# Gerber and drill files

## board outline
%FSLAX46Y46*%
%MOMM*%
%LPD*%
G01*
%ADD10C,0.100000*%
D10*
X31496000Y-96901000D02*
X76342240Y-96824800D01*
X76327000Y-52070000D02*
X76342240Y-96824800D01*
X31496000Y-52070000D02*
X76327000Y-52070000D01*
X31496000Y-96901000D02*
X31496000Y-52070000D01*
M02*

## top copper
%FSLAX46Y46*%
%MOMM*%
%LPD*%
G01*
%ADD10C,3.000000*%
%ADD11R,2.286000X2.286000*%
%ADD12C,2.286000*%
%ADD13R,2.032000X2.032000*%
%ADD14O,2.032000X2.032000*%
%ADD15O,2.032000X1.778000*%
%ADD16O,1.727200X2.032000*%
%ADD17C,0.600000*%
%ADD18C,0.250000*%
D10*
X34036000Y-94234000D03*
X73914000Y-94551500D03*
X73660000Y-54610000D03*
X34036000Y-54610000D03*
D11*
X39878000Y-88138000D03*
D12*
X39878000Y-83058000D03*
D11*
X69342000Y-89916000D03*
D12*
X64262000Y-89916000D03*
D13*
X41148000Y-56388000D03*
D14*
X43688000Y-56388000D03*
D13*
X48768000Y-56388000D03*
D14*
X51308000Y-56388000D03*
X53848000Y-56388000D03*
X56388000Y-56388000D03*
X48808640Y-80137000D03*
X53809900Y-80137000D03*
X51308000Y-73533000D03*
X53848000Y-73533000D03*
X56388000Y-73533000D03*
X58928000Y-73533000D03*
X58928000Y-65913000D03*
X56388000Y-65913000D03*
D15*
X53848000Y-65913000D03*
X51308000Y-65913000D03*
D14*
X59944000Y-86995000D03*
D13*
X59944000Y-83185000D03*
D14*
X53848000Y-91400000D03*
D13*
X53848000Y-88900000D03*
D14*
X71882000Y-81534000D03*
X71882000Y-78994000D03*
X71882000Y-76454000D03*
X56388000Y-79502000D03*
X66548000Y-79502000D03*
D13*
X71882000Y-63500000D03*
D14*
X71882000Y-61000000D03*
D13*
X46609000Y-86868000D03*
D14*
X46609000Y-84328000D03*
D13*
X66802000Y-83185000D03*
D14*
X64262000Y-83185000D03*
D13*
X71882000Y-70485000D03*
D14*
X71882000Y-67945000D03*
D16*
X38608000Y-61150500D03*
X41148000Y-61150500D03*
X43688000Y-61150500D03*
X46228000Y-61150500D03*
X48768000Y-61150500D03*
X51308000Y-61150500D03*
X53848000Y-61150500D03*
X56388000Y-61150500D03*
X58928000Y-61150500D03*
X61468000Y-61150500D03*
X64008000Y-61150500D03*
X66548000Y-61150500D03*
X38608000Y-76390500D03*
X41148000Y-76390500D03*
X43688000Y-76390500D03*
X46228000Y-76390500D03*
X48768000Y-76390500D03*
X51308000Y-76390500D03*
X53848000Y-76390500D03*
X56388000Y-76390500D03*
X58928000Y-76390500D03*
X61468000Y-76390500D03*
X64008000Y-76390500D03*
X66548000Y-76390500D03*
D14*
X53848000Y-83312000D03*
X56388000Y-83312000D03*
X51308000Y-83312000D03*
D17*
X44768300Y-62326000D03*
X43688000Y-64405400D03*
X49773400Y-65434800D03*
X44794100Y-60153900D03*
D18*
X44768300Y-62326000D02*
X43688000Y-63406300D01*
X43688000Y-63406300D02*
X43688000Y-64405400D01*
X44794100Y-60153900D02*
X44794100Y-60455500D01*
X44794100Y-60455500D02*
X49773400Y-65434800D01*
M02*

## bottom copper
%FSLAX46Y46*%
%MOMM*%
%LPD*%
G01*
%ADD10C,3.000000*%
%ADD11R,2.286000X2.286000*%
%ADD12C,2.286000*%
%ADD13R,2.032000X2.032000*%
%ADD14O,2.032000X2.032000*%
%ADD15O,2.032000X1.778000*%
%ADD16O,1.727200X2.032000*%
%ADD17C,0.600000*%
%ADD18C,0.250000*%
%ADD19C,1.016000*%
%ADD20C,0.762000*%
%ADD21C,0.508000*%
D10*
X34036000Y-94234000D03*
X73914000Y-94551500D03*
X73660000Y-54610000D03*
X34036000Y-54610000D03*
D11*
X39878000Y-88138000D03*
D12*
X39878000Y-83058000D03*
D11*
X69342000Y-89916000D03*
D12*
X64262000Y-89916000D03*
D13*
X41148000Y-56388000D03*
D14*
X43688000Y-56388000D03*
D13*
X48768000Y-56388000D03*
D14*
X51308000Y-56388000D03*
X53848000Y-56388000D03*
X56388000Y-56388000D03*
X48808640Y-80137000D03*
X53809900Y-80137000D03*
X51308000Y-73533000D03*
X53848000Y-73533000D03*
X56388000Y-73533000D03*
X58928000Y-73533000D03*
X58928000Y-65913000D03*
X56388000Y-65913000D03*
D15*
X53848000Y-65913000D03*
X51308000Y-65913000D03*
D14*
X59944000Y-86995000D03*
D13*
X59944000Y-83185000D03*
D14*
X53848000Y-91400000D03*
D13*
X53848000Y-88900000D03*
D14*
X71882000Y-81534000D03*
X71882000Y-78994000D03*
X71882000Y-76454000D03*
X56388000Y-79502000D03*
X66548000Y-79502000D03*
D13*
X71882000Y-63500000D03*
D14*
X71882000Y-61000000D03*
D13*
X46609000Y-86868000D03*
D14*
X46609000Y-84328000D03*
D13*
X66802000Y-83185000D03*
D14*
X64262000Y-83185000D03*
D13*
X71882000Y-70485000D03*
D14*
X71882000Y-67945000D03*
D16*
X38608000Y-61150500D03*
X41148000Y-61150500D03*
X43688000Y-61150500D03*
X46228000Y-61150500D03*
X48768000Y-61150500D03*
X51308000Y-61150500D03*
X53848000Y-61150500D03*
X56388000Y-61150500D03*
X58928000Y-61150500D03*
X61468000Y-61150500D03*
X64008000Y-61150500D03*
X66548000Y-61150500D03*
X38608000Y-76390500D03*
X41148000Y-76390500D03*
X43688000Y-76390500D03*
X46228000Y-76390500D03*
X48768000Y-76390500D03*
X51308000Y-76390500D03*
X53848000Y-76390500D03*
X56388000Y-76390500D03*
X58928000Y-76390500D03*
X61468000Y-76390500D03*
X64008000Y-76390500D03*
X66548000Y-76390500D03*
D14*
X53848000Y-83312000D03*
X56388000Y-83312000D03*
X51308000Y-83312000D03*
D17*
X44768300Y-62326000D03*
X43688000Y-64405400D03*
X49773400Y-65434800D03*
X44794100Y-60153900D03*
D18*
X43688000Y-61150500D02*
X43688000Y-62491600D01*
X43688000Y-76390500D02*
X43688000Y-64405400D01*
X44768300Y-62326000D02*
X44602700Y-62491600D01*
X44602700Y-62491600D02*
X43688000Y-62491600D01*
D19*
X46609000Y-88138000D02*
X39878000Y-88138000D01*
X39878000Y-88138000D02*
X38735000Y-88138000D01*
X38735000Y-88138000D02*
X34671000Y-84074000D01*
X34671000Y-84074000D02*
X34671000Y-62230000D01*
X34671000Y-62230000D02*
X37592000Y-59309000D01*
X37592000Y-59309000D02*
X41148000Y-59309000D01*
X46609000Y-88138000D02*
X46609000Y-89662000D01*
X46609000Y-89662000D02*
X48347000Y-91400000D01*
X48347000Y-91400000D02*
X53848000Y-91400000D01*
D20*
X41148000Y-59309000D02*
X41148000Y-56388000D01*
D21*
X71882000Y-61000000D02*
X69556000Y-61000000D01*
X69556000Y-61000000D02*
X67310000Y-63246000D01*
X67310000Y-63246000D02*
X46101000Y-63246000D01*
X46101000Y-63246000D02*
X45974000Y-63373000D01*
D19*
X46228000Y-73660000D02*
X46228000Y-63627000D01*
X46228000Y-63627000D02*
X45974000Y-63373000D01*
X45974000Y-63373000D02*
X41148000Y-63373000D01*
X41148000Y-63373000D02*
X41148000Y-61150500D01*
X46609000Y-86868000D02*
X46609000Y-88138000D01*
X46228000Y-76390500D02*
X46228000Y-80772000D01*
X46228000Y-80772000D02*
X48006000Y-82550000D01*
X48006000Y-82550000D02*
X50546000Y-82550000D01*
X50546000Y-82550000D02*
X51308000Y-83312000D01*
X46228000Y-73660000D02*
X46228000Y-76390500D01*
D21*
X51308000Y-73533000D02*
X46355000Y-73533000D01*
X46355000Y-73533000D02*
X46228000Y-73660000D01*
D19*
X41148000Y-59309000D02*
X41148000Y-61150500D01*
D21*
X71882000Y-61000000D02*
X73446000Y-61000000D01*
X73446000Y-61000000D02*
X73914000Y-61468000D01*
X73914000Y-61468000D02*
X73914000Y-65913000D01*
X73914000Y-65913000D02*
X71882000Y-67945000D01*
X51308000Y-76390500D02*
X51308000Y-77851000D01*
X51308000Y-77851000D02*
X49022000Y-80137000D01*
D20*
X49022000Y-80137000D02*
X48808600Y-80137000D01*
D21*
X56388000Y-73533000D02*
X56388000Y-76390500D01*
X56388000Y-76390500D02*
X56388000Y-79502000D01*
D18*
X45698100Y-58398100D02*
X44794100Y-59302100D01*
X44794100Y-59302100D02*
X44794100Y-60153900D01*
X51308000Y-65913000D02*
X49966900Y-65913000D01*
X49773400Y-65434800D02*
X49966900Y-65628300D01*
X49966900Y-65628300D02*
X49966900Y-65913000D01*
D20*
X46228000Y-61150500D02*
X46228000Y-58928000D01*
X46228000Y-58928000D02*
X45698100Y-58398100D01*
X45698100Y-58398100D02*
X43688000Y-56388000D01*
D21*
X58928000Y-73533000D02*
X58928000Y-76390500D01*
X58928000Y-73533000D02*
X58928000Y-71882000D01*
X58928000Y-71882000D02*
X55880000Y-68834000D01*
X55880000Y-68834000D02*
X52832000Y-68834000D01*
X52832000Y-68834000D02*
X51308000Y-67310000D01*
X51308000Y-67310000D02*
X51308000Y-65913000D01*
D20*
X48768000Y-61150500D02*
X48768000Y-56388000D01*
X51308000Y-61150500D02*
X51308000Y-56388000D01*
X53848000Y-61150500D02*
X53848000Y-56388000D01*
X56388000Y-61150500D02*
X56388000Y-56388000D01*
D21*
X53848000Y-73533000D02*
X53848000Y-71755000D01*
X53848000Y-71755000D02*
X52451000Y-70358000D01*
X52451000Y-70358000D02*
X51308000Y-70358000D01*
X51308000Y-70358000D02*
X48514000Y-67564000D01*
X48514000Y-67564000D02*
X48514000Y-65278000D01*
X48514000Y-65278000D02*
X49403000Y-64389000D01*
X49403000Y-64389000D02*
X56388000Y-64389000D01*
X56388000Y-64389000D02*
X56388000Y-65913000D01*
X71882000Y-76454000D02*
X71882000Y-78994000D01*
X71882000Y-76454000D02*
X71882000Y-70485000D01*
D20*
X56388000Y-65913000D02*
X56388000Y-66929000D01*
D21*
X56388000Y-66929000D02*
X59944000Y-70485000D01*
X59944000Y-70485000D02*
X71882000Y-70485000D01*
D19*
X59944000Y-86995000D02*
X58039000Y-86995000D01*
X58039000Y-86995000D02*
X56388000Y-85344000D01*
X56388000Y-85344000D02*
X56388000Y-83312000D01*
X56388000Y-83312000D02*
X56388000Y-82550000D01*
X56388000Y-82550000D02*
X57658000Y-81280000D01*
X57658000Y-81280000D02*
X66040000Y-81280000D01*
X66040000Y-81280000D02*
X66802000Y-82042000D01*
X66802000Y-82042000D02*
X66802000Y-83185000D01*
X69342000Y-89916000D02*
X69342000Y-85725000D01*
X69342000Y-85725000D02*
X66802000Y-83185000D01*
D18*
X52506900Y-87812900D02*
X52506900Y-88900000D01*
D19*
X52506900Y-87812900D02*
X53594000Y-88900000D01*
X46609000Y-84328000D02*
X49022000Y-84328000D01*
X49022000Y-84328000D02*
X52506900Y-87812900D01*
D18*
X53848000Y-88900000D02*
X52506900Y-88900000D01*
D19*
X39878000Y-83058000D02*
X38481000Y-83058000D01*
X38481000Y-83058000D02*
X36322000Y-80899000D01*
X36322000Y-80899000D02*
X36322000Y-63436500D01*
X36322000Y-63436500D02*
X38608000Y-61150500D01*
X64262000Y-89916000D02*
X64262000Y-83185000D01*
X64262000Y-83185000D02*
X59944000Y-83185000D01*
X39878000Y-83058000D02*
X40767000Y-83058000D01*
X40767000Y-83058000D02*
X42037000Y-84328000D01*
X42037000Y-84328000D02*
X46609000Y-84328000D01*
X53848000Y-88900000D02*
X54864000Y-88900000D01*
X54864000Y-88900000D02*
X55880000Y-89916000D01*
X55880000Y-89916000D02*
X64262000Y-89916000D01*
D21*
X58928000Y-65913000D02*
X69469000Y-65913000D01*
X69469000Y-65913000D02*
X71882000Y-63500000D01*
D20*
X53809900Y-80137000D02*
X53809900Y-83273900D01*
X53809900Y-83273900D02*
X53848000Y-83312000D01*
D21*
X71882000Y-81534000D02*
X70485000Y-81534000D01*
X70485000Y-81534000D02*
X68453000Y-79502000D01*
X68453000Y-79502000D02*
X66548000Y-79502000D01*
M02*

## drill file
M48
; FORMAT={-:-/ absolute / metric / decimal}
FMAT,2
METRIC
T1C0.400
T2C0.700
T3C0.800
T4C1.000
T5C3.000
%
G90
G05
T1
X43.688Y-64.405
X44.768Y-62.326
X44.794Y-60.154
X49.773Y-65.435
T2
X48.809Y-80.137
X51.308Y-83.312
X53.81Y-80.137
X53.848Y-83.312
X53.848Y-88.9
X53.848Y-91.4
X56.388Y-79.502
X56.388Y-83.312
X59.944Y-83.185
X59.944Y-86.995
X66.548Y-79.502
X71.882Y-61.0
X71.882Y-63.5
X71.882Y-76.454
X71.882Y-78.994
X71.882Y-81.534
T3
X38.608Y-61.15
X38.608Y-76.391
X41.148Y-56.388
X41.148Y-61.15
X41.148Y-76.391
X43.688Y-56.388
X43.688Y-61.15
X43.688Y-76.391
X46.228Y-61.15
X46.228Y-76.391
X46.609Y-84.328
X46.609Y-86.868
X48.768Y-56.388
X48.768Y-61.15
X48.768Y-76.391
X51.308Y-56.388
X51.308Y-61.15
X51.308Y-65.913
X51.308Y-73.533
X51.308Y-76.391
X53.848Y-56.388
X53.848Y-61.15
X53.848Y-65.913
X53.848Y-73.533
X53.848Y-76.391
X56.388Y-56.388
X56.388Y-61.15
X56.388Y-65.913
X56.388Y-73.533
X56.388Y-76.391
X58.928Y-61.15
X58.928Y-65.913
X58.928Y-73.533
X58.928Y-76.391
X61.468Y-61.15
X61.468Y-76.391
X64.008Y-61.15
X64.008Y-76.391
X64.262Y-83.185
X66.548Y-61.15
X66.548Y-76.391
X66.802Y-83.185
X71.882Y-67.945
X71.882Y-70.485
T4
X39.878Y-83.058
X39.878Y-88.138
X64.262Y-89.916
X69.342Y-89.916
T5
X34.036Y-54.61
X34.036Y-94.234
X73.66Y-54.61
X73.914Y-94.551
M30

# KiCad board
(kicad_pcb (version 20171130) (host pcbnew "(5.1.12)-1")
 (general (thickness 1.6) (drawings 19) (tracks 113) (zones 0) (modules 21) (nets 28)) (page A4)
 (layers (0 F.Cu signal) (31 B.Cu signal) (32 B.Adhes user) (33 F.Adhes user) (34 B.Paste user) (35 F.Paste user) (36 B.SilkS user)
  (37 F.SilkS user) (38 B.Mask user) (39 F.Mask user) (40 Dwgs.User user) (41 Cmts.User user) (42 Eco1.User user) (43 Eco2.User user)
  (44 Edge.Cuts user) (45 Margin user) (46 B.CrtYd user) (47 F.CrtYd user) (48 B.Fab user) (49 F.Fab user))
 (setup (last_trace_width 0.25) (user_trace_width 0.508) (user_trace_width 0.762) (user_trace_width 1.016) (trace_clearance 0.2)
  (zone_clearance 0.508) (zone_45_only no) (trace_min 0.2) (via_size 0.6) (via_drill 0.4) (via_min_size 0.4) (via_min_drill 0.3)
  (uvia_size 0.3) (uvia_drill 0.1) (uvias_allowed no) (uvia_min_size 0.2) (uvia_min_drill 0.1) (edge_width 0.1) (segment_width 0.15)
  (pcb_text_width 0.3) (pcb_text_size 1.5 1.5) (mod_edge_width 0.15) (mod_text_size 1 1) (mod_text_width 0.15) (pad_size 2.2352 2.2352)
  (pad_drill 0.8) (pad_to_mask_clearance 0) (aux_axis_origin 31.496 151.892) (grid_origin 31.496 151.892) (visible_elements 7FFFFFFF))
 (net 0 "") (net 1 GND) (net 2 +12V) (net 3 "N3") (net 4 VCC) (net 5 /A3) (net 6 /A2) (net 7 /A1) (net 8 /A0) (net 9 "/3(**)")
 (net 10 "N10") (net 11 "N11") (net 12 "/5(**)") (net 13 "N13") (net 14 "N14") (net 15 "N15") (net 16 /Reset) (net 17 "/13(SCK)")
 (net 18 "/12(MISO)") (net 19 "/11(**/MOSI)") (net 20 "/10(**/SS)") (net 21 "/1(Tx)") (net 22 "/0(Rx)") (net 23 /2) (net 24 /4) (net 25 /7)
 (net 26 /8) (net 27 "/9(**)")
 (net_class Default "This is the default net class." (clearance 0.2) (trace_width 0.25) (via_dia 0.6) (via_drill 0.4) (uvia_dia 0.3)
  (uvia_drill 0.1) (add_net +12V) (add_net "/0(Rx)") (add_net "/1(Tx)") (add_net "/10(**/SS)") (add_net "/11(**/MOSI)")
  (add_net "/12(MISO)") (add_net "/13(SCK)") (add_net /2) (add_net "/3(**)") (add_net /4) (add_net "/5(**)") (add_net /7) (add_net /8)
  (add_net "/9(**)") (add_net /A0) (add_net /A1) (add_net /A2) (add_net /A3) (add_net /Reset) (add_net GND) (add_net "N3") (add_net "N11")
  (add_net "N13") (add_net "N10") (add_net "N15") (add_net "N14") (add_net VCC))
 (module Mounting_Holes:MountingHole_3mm (layer F.Cu) (at 34.036 94.234)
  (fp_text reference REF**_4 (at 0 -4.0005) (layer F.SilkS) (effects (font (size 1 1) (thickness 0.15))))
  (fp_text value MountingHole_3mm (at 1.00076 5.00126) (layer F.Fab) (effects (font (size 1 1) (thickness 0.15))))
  (pad 1 thru_hole circle (at 0 0) (size 3 3) (drill 3) (layers *.Cu *.Mask)))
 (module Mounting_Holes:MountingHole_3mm (layer F.Cu) (at 73.914 94.5515)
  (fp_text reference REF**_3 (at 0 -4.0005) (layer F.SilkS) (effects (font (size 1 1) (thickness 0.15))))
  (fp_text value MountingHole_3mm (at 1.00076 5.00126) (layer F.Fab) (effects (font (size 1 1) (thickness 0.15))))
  (pad 1 thru_hole circle (at 0 0) (size 3 3) (drill 3) (layers *.Cu *.Mask)))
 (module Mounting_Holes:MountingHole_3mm (layer F.Cu) (at 73.66 54.61)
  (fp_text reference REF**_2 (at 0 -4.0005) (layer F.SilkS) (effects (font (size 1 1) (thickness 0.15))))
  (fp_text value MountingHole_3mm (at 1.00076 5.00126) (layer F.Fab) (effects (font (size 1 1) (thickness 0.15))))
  (pad 1 thru_hole circle (at 0 0) (size 3 3) (drill 3) (layers *.Cu *.Mask)))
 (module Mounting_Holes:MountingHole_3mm (layer F.Cu) (at 34.036 54.61)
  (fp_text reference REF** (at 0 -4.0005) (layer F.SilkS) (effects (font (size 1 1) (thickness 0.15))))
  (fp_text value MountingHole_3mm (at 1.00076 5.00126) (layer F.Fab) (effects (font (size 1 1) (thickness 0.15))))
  (pad 1 thru_hole circle (at 0 0) (size 3 3) (drill 3) (layers *.Cu *.Mask)))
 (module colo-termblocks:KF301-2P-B (layer F.Cu) (at 39.878 85.598 90)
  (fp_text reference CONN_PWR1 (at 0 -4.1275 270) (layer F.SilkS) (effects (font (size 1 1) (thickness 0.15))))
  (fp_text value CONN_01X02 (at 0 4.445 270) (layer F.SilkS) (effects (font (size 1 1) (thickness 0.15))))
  (pad 1 thru_hole rect (at -2.54 0 90) (size 2.286 2.286) (drill 1) (layers B.Cu B.Mask) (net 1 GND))
  (pad 2 thru_hole circle (at 2.54 0 90) (size 2.286 2.286) (drill 1) (layers B.Cu B.Mask) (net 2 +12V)))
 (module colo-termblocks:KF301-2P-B (layer F.Cu) (at 66.802 89.916 180)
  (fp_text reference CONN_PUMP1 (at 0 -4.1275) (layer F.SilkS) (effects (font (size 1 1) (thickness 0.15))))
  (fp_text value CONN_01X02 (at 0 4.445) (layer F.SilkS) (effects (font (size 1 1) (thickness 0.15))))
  (pad 1 thru_hole rect (at -2.54 0 180) (size 2.286 2.286) (drill 1) (layers B.Cu B.Mask) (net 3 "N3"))
  (pad 2 thru_hole circle (at 2.54 0 180) (size 2.286 2.286) (drill 1) (layers B.Cu B.Mask) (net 2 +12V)))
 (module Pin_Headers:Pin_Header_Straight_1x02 (layer F.Cu) (at 41.148 56.388 90)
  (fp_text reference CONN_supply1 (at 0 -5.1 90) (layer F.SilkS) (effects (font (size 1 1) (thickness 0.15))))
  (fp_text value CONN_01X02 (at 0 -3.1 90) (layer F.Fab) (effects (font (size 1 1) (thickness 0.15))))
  (pad 1 thru_hole rect (at 0 0 90) (size 2.032 2.032) (drill 0.8) (layers B.Cu B.Mask) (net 1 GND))
  (pad 2 thru_hole oval (at 0 2.54 90) (size 2.032 2.032) (drill 0.8) (layers B.Cu B.Mask) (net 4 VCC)))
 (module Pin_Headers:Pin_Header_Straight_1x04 (layer F.Cu) (at 48.768 56.388 90)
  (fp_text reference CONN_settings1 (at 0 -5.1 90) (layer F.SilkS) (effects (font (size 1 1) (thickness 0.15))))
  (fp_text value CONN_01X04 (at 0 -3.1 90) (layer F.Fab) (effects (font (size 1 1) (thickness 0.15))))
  (pad 1 thru_hole rect (at 0 0 90) (size 2.032 2.032) (drill 0.8) (layers B.Cu B.Mask) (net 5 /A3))
  (pad 2 thru_hole oval (at 0 2.54 90) (size 2.032 2.032) (drill 0.8) (layers B.Cu B.Mask) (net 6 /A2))
  (pad 3 thru_hole oval (at 0 5.08 90) (size 2.032 2.032) (drill 0.8) (layers B.Cu B.Mask) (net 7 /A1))
  (pad 4 thru_hole oval (at 0 7.62 90) (size 2.032 2.032) (drill 0.8) (layers B.Cu B.Mask) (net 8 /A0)))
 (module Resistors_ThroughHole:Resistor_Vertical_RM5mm (layer F.Cu) (at 51.308 80.137)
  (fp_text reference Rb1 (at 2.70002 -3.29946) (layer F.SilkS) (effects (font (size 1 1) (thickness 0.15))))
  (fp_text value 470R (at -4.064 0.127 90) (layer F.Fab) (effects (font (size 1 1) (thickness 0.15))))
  (pad 1 thru_hole oval (at -2.49936 0) (size 2.032 2.032) (drill 0.7) (layers B.Cu B.Mask) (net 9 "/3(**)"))
  (pad 2 thru_hole oval (at 2.5019 0) (size 2.032 2.032) (drill 0.7) (layers B.Cu B.Mask) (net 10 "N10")))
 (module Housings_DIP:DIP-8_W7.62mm (layer F.Cu) (at 51.308 73.533 90)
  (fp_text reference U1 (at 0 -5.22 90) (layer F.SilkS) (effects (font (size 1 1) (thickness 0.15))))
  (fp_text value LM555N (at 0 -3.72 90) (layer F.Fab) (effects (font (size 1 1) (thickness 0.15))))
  (pad 1 thru_hole oval (at 0 0 90) (size 2.032 2.032) (drill 0.8) (layers B.Cu B.Mask) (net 1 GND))
  (pad 2 thru_hole oval (at 0 2.54 90) (size 2.032 2.032) (drill 0.8) (layers B.Cu B.Mask) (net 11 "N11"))
  (pad 3 thru_hole oval (at 0 5.08 90) (size 2.032 2.032) (drill 0.8) (layers B.Cu B.Mask) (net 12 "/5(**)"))
  (pad 4 thru_hole oval (at 0 7.62 90) (size 2.032 2.032) (drill 0.8) (layers B.Cu B.Mask) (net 4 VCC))
  (pad 5 thru_hole oval (at 7.62 7.62 90) (size 2.032 2.032) (drill 0.8) (layers B.Cu B.Mask) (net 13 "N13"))
  (pad 6 thru_hole oval (at 7.62 5.08 90) (size 2.032 2.032) (drill 0.8) (layers B.Cu B.Mask) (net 11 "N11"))
  (pad 7 thru_hole oval (at 7.62 2.54 90) (size 1.778 2.032) (drill 0.8) (layers B.Cu B.Mask) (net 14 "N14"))
  (pad 8 thru_hole oval (at 7.62 0 90) (size 1.778 2.032) (drill 0.8) (layers B.Cu B.Mask) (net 4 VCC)))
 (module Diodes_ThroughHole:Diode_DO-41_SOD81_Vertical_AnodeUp (layer F.Cu) (at 59.944 83.185 270)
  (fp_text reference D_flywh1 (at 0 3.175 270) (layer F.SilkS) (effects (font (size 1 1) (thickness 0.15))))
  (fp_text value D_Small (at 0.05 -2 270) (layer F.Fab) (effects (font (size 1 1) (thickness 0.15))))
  (pad 2 thru_hole oval (at 3.81 0 270) (size 2.032 2.032) (drill 0.7) (layers B.Cu B.Mask) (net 3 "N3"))
  (pad 1 thru_hole rect (at 0 0 270) (size 2.032 2.032) (drill 0.7) (layers B.Cu B.Mask) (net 2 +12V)))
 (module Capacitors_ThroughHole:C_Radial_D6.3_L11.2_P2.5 (layer F.Cu) (at 53.848 88.9 270)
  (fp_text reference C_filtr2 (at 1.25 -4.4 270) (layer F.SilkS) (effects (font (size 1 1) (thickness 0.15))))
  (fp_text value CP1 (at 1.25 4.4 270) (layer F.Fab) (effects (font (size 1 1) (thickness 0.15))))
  (pad 2 thru_hole oval (at 2.5 0 270) (size 2.032 2.032) (drill 0.7) (layers B.Cu B.Mask) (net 1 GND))
  (pad 1 thru_hole rect (at 0 0 270) (size 2.032 2.032) (drill 0.7) (layers B.Cu B.Mask) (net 2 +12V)))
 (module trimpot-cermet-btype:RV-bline (layer F.Cu) (at 71.882 78.994 90)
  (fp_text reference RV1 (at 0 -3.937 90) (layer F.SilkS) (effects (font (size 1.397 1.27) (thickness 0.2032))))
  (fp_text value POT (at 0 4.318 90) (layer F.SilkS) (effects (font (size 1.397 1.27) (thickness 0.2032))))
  (pad 1 thru_hole oval (at -2.54 0 90) (size 2.032 2.032) (drill 0.7) (layers B.Cu B.Mask) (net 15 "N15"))
  (pad 2 thru_hole oval (at 0 0 90) (size 2.032 2.032) (drill 0.7) (layers B.Cu B.Mask) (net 11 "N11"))
  (pad 3 thru_hole oval (at 2.54 0 90) (size 2.032 2.032) (drill 0.7) (layers B.Cu B.Mask) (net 11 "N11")))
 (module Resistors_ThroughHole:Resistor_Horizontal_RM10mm (layer F.Cu) (at 61.468 79.502)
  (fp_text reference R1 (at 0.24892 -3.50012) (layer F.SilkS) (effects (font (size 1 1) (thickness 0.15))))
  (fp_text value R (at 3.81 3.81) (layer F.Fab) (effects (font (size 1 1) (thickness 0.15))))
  (pad 1 thru_hole oval (at -5.08 0) (size 2.032 2.032) (drill 0.7) (layers B.Cu B.Mask) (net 12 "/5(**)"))
  (pad 2 thru_hole oval (at 5.08 0) (size 2.032 2.032) (drill 0.7) (layers B.Cu B.Mask) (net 15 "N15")))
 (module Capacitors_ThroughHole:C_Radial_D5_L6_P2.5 (layer F.Cu) (at 71.882 63.5 90)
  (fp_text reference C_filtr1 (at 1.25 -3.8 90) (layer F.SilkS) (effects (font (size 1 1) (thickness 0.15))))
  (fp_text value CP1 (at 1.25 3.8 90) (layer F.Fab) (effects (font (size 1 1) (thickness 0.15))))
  (pad 1 thru_hole rect (at 0 0 90) (size 2.032 2.032) (drill 0.7) (layers B.Cu B.Mask) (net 13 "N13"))
  (pad 2 thru_hole oval (at 2.5 0 90) (size 2.032 2.032) (drill 0.7) (layers B.Cu B.Mask) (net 1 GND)))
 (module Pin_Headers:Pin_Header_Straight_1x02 (layer F.Cu) (at 46.609 86.868 180)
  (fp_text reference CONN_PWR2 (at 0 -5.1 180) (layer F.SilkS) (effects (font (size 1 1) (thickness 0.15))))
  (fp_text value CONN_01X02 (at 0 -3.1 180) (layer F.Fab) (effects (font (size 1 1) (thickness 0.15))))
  (pad 1 thru_hole rect (at 0 0 180) (size 2.032 2.032) (drill 0.8) (layers B.Cu B.Mask) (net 1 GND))
  (pad 2 thru_hole oval (at 0 2.54 180) (size 2.032 2.032) (drill 0.8) (layers B.Cu B.Mask) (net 2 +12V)))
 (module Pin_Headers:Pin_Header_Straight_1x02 (layer F.Cu) (at 66.802 83.185 270)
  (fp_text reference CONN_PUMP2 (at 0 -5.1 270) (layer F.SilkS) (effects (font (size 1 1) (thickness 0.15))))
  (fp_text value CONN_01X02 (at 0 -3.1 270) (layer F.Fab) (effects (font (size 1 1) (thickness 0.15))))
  (pad 1 thru_hole rect (at 0 0 270) (size 2.032 2.032) (drill 0.8) (layers B.Cu B.Mask) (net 3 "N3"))
  (pad 2 thru_hole oval (at 0 2.54 270) (size 2.032 2.032) (drill 0.8) (layers B.Cu B.Mask) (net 2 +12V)))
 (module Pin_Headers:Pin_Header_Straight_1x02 (layer F.Cu) (at 71.882 70.485 180)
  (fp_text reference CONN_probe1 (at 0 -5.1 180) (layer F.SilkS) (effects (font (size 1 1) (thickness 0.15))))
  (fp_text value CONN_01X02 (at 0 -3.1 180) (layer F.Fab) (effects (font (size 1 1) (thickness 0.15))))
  (pad 1 thru_hole rect (at 0 0 180) (size 2.032 2.032) (drill 0.8) (layers B.Cu B.Mask) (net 11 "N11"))
  (pad 2 thru_hole oval (at 0 2.54 180) (size 2.032 2.032) (drill 0.8) (layers B.Cu B.Mask) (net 1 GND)))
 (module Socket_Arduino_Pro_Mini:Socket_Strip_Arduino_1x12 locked (layer F.Cu) (at 38.608 61.1505)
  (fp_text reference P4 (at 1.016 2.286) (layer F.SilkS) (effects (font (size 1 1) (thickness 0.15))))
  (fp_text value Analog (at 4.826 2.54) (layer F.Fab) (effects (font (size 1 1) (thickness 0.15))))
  (pad 1 thru_hole oval (at 0 0) (size 1.7272 2.032) (drill 0.8) (layers B.Cu B.Mask) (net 2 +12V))
  (pad 2 thru_hole oval (at 2.54 0) (size 1.7272 2.032) (drill 0.8) (layers B.Cu B.Mask) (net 1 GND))
  (pad 3 thru_hole oval (at 5.08 0) (size 1.7272 2.032) (drill 0.8) (layers B.Cu B.Mask) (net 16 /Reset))
  (pad 4 thru_hole oval (at 7.62 0) (size 1.7272 2.032) (drill 0.8) (layers B.Cu B.Mask) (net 4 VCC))
  (pad 5 thru_hole oval (at 10.16 0) (size 1.7272 2.032) (drill 0.8) (layers B.Cu B.Mask) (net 5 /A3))
  (pad 6 thru_hole oval (at 12.7 0) (size 1.7272 2.032) (drill 0.8) (layers B.Cu B.Mask) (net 6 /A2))
  (pad 7 thru_hole oval (at 15.24 0) (size 1.7272 2.032) (drill 0.8) (layers B.Cu B.Mask) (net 7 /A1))
  (pad 8 thru_hole oval (at 17.78 0) (size 1.7272 2.032) (drill 0.8) (layers B.Cu B.Mask) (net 8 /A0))
  (pad 9 thru_hole oval (at 20.32 0) (size 1.7272 2.032) (drill 0.8) (layers B.Cu B.Mask) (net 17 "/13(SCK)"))
  (pad 10 thru_hole oval (at 22.86 0) (size 1.7272 2.032) (drill 0.8) (layers B.Cu B.Mask) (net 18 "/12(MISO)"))
  (pad 11 thru_hole oval (at 25.4 0) (size 1.7272 2.032) (drill 0.8) (layers B.Cu B.Mask) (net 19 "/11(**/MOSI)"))
  (pad 12 thru_hole oval (at 27.94 0) (size 1.7272 2.032) (drill 0.8) (layers B.Cu B.Mask) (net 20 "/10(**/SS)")))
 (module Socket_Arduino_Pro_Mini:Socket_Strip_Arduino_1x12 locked (layer F.Cu) (at 38.608 76.3905)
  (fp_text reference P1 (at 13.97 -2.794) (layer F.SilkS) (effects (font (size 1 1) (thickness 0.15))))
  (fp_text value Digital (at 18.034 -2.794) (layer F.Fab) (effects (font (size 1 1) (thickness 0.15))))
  (pad 1 thru_hole oval (at 0 0) (size 1.7272 2.032) (drill 0.8) (layers B.Cu B.Mask) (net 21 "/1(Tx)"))
  (pad 2 thru_hole oval (at 2.54 0) (size 1.7272 2.032) (drill 0.8) (layers B.Cu B.Mask) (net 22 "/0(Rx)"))
  (pad 3 thru_hole oval (at 5.08 0) (size 1.7272 2.032) (drill 0.8) (layers B.Cu B.Mask) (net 16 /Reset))
  (pad 4 thru_hole oval (at 7.62 0) (size 1.7272 2.032) (drill 0.8) (layers B.Cu B.Mask) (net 1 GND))
  (pad 5 thru_hole oval (at 10.16 0) (size 1.7272 2.032) (drill 0.8) (layers B.Cu B.Mask) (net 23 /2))
  (pad 6 thru_hole oval (at 12.7 0) (size 1.7272 2.032) (drill 0.8) (layers B.Cu B.Mask) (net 9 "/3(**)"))
  (pad 7 thru_hole oval (at 15.24 0) (size 1.7272 2.032) (drill 0.8) (layers B.Cu B.Mask) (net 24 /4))
  (pad 8 thru_hole oval (at 17.78 0) (size 1.7272 2.032) (drill 0.8) (layers B.Cu B.Mask) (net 12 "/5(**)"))
  (pad 9 thru_hole oval (at 20.32 0) (size 1.7272 2.032) (drill 0.8) (layers B.Cu B.Mask) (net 4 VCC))
  (pad 10 thru_hole oval (at 22.86 0) (size 1.7272 2.032) (drill 0.8) (layers B.Cu B.Mask) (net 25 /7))
  (pad 11 thru_hole oval (at 25.4 0) (size 1.7272 2.032) (drill 0.8) (layers B.Cu B.Mask) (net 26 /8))
  (pad 12 thru_hole oval (at 27.94 0) (size 1.7272 2.032) (drill 0.8) (layers B.Cu B.Mask) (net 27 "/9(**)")))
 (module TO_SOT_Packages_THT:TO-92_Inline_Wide (layer F.Cu) (at 51.308 83.312)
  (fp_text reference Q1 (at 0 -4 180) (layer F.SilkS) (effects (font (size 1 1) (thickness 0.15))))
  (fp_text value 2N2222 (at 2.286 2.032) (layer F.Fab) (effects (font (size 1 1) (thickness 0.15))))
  (pad 2 thru_hole oval (at 2.54 0) (size 2.032 2.032) (drill 0.7) (layers B.Cu B.Mask) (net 10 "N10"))
  (pad 3 thru_hole oval (at 5.08 0) (size 2.032 2.032) (drill 0.7) (layers B.Cu B.Mask) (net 3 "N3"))
  (pad 1 thru_hole oval (at 0 0) (size 2.032 2.032) (drill 0.7) (layers B.Cu B.Mask) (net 1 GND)))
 (gr_line (start 31.496 96.901) (end 76.34224 96.8248) (angle 90) (layer Edge.Cuts) (width 0.1))
 (gr_line (start 76.327 52.07) (end 76.34224 96.8248) (angle 90) (layer Edge.Cuts) (width 0.1))
 (gr_line (start 31.496 52.07) (end 76.327 52.07) (angle 90) (layer Edge.Cuts) (width 0.1))
 (gr_line (start 31.496 96.901) (end 31.496 52.07) (angle 90) (layer Edge.Cuts) (width 0.1))
 (segment (start 43.688 61.1505) (end 43.688 62.4916) (width 0.25) (layer B.Cu) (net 16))
 (segment (start 44.7683 62.326) (end 43.688 63.4063) (width 0.25) (layer F.Cu) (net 16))
 (segment (start 43.688 63.4063) (end 43.688 64.4054) (width 0.25) (layer F.Cu) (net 16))
 (segment (start 43.688 76.3905) (end 43.688 64.4054) (width 0.25) (layer B.Cu) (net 16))
 (segment (start 44.7683 62.326) (end 44.6027 62.4916) (width 0.25) (layer B.Cu) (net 16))
 (segment (start 44.6027 62.4916) (end 43.688 62.4916) (width 0.25) (layer B.Cu) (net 16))
 (via (at 44.7683 62.326) (size 0.6) (layers F.Cu B.Cu) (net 16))
 (via (at 43.688 64.4054) (size 0.6) (layers F.Cu B.Cu) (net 16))
 (segment (start 46.609 88.138) (end 39.878 88.138) (width 1.016) (layer B.Cu) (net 1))
 (segment (start 39.878 88.138) (end 38.735 88.138) (width 1.016) (layer B.Cu) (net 1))
 (segment (start 38.735 88.138) (end 34.671 84.074) (width 1.016) (layer B.Cu) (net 1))
 (segment (start 34.671 84.074) (end 34.671 62.23) (width 1.016) (layer B.Cu) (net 1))
 (segment (start 34.671 62.23) (end 37.592 59.309) (width 1.016) (layer B.Cu) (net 1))
 (segment (start 37.592 59.309) (end 41.148 59.309) (width 1.016) (layer B.Cu) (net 1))
 (segment (start 46.609 88.138) (end 46.609 89.662) (width 1.016) (layer B.Cu) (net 1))
 (segment (start 46.609 89.662) (end 48.347 91.4) (width 1.016) (layer B.Cu) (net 1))
 (segment (start 48.347 91.4) (end 53.848 91.4) (width 1.016) (layer B.Cu) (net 1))
 (segment (start 41.148 59.309) (end 41.148 56.388) (width 0.762) (layer B.Cu) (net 1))
 (segment (start 71.882 61) (end 69.556 61) (width 0.508) (layer B.Cu) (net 1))
 (segment (start 69.556 61) (end 67.31 63.246) (width 0.508) (layer B.Cu) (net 1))
 (segment (start 67.31 63.246) (end 46.101 63.246) (width 0.508) (layer B.Cu) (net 1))
 (segment (start 46.101 63.246) (end 45.974 63.373) (width 0.508) (layer B.Cu) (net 1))
 (segment (start 46.228 73.66) (end 46.228 63.627) (width 1.016) (layer B.Cu) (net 1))
 (segment (start 46.228 63.627) (end 45.974 63.373) (width 1.016) (layer B.Cu) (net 1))
 (segment (start 45.974 63.373) (end 41.148 63.373) (width 1.016) (layer B.Cu) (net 1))
 (segment (start 41.148 63.373) (end 41.148 61.1505) (width 1.016) (layer B.Cu) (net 1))
 (segment (start 46.609 86.868) (end 46.609 88.138) (width 1.016) (layer B.Cu) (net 1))
 (segment (start 46.228 76.3905) (end 46.228 80.772) (width 1.016) (layer B.Cu) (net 1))
 (segment (start 46.228 80.772) (end 48.006 82.55) (width 1.016) (layer B.Cu) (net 1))
 (segment (start 48.006 82.55) (end 50.546 82.55) (width 1.016) (layer B.Cu) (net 1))
 (segment (start 50.546 82.55) (end 51.308 83.312) (width 1.016) (layer B.Cu) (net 1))
 (segment (start 46.228 73.66) (end 46.228 76.3905) (width 1.016) (layer B.Cu) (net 1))
 (segment (start 51.308 73.533) (end 46.355 73.533) (width 0.508) (layer B.Cu) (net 1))
 (segment (start 46.355 73.533) (end 46.228 73.66) (width 0.508) (layer B.Cu) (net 1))
 (segment (start 41.148 59.309) (end 41.148 61.1505) (width 1.016) (layer B.Cu) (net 1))
 (segment (start 71.882 61) (end 73.446 61) (width 0.508) (layer B.Cu) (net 1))
 (segment (start 73.446 61) (end 73.914 61.468) (width 0.508) (layer B.Cu) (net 1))
 (segment (start 73.914 61.468) (end 73.914 65.913) (width 0.508) (layer B.Cu) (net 1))
 (segment (start 73.914 65.913) (end 71.882 67.945) (width 0.508) (layer B.Cu) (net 1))
 (segment (start 51.308 76.3905) (end 51.308 77.851) (width 0.508) (layer B.Cu) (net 9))
 (segment (start 51.308 77.851) (end 49.022 80.137) (width 0.508) (layer B.Cu) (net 9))
 (segment (start 49.022 80.137) (end 48.8086 80.137) (width 0.762) (layer B.Cu) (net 9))
 (segment (start 56.388 73.533) (end 56.388 76.3905) (width 0.508) (layer B.Cu) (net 12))
 (segment (start 56.388 76.3905) (end 56.388 79.502) (width 0.508) (layer B.Cu) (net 12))
 (segment (start 44.7941 60.1539) (end 44.7941 60.4555) (width 0.25) (layer F.Cu) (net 4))
 (segment (start 44.7941 60.4555) (end 49.7734 65.4348) (width 0.25) (layer F.Cu) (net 4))
 (segment (start 45.6981 58.3981) (end 44.7941 59.3021) (width 0.25) (layer B.Cu) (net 4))
 (segment (start 44.7941 59.3021) (end 44.7941 60.1539) (width 0.25) (layer B.Cu) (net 4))
 (segment (start 51.308 65.913) (end 49.9669 65.913) (width 0.25) (layer B.Cu) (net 4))
 (segment (start 49.7734 65.4348) (end 49.9669 65.6283) (width 0.25) (layer B.Cu) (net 4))
 (segment (start 49.9669 65.6283) (end 49.9669 65.913) (width 0.25) (layer B.Cu) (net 4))
 (segment (start 46.228 61.1505) (end 46.228 58.928) (width 0.762) (layer B.Cu) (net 4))
 (segment (start 46.228 58.928) (end 45.6981 58.3981) (width 0.762) (layer B.Cu) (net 4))
 (segment (start 45.6981 58.3981) (end 43.688 56.388) (width 0.762) (layer B.Cu) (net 4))
 (segment (start 58.928 73.533) (end 58.928 76.3905) (width 0.508) (layer B.Cu) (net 4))
 (segment (start 58.928 73.533) (end 58.928 71.882) (width 0.508) (layer B.Cu) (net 4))
 (segment (start 58.928 71.882) (end 55.88 68.834) (width 0.508) (layer B.Cu) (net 4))
 (segment (start 55.88 68.834) (end 52.832 68.834) (width 0.508) (layer B.Cu) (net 4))
 (segment (start 52.832 68.834) (end 51.308 67.31) (width 0.508) (layer B.Cu) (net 4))
 (segment (start 51.308 67.31) (end 51.308 65.913) (width 0.508) (layer B.Cu) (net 4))
 (via (at 49.7734 65.4348) (size 0.6) (layers F.Cu B.Cu) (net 4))
 (via (at 44.7941 60.1539) (size 0.6) (layers F.Cu B.Cu) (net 4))
 (segment (start 48.768 61.1505) (end 48.768 56.388) (width 0.762) (layer B.Cu) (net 5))
 (segment (start 51.308 61.1505) (end 51.308 56.388) (width 0.762) (layer B.Cu) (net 6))
 (segment (start 53.848 61.1505) (end 53.848 56.388) (width 0.762) (layer B.Cu) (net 7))
 (segment (start 56.388 61.1505) (end 56.388 56.388) (width 0.762) (layer B.Cu) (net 8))
 (segment (start 53.848 73.533) (end 53.848 71.755) (width 0.508) (layer B.Cu) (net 11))
 (segment (start 53.848 71.755) (end 52.451 70.358) (width 0.508) (layer B.Cu) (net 11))
 (segment (start 52.451 70.358) (end 51.308 70.358) (width 0.508) (layer B.Cu) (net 11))
 (segment (start 51.308 70.358) (end 48.514 67.564) (width 0.508) (layer B.Cu) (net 11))
 (segment (start 48.514 67.564) (end 48.514 65.278) (width 0.508) (layer B.Cu) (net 11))
 (segment (start 48.514 65.278) (end 49.403 64.389) (width 0.508) (layer B.Cu) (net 11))
 (segment (start 49.403 64.389) (end 56.388 64.389) (width 0.508) (layer B.Cu) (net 11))
 (segment (start 56.388 64.389) (end 56.388 65.913) (width 0.508) (layer B.Cu) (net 11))
 (segment (start 71.882 76.454) (end 71.882 78.994) (width 0.508) (layer B.Cu) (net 11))
 (segment (start 71.882 76.454) (end 71.882 70.485) (width 0.508) (layer B.Cu) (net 11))
 (segment (start 56.388 65.913) (end 56.388 66.929) (width 0.762) (layer B.Cu) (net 11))
 (segment (start 56.388 66.929) (end 59.944 70.485) (width 0.508) (layer B.Cu) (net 11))
 (segment (start 59.944 70.485) (end 71.882 70.485) (width 0.508) (layer B.Cu) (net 11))
 (segment (start 59.944 86.995) (end 58.039 86.995) (width 1.016) (layer B.Cu) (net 3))
 (segment (start 58.039 86.995) (end 56.388 85.344) (width 1.016) (layer B.Cu) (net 3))
 (segment (start 56.388 85.344) (end 56.388 83.312) (width 1.016) (layer B.Cu) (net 3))
 (segment (start 56.388 83.312) (end 56.388 82.55) (width 1.016) (layer B.Cu) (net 3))
 (segment (start 56.388 82.55) (end 57.658 81.28) (width 1.016) (layer B.Cu) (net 3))
 (segment (start 57.658 81.28) (end 66.04 81.28) (width 1.016) (layer B.Cu) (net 3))
 (segment (start 66.04 81.28) (end 66.802 82.042) (width 1.016) (layer B.Cu) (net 3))
 (segment (start 66.802 82.042) (end 66.802 83.185) (width 1.016) (layer B.Cu) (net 3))
 (segment (start 69.342 89.916) (end 69.342 85.725) (width 1.016) (layer B.Cu) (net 3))
 (segment (start 69.342 85.725) (end 66.802 83.185) (width 1.016) (layer B.Cu) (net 3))
 (segment (start 52.5069 87.8129) (end 52.5069 88.9) (width 0.25) (layer B.Cu) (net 2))
 (segment (start 52.5069 87.8129) (end 53.594 88.9) (width 1.016) (layer B.Cu) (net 2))
 (segment (start 46.609 84.328) (end 49.022 84.328) (width 1.016) (layer B.Cu) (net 2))
 (segment (start 49.022 84.328) (end 52.5069 87.8129) (width 1.016) (layer B.Cu) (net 2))
 (segment (start 53.848 88.9) (end 52.5069 88.9) (width 0.25) (layer B.Cu) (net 2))
 (segment (start 39.878 83.058) (end 38.481 83.058) (width 1.016) (layer B.Cu) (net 2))
 (segment (start 38.481 83.058) (end 36.322 80.899) (width 1.016) (layer B.Cu) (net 2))
 (segment (start 36.322 80.899) (end 36.322 63.4365) (width 1.016) (layer B.Cu) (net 2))
 (segment (start 36.322 63.4365) (end 38.608 61.1505) (width 1.016) (layer B.Cu) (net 2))
 (segment (start 64.262 89.916) (end 64.262 83.185) (width 1.016) (layer B.Cu) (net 2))
 (segment (start 64.262 83.185) (end 59.944 83.185) (width 1.016) (layer B.Cu) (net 2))
 (segment (start 39.878 83.058) (end 40.767 83.058) (width 1.016) (layer B.Cu) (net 2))
 (segment (start 40.767 83.058) (end 42.037 84.328) (width 1.016) (layer B.Cu) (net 2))
 (segment (start 42.037 84.328) (end 46.609 84.328) (width 1.016) (layer B.Cu) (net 2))
 (segment (start 53.848 88.9) (end 54.864 88.9) (width 1.016) (layer B.Cu) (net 2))
 (segment (start 54.864 88.9) (end 55.88 89.916) (width 1.016) (layer B.Cu) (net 2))
 (segment (start 55.88 89.916) (end 64.262 89.916) (width 1.016) (layer B.Cu) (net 2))
 (segment (start 58.928 65.913) (end 69.469 65.913) (width 0.508) (layer B.Cu) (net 13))
 (segment (start 69.469 65.913) (end 71.882 63.5) (width 0.508) (layer B.Cu) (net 13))
 (segment (start 53.8099 80.137) (end 53.8099 83.2739) (width 0.762) (layer B.Cu) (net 10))
 (segment (start 53.8099 83.2739) (end 53.848 83.312) (width 0.762) (layer B.Cu) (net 10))
 (segment (start 71.882 81.534) (end 70.485 81.534) (width 0.508) (layer B.Cu) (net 15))
 (segment (start 70.485 81.534) (end 68.453 79.502) (width 0.508) (layer B.Cu) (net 15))
 (segment (start 68.453 79.502) (end 66.548 79.502) (width 0.508) (layer B.Cu) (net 15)))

